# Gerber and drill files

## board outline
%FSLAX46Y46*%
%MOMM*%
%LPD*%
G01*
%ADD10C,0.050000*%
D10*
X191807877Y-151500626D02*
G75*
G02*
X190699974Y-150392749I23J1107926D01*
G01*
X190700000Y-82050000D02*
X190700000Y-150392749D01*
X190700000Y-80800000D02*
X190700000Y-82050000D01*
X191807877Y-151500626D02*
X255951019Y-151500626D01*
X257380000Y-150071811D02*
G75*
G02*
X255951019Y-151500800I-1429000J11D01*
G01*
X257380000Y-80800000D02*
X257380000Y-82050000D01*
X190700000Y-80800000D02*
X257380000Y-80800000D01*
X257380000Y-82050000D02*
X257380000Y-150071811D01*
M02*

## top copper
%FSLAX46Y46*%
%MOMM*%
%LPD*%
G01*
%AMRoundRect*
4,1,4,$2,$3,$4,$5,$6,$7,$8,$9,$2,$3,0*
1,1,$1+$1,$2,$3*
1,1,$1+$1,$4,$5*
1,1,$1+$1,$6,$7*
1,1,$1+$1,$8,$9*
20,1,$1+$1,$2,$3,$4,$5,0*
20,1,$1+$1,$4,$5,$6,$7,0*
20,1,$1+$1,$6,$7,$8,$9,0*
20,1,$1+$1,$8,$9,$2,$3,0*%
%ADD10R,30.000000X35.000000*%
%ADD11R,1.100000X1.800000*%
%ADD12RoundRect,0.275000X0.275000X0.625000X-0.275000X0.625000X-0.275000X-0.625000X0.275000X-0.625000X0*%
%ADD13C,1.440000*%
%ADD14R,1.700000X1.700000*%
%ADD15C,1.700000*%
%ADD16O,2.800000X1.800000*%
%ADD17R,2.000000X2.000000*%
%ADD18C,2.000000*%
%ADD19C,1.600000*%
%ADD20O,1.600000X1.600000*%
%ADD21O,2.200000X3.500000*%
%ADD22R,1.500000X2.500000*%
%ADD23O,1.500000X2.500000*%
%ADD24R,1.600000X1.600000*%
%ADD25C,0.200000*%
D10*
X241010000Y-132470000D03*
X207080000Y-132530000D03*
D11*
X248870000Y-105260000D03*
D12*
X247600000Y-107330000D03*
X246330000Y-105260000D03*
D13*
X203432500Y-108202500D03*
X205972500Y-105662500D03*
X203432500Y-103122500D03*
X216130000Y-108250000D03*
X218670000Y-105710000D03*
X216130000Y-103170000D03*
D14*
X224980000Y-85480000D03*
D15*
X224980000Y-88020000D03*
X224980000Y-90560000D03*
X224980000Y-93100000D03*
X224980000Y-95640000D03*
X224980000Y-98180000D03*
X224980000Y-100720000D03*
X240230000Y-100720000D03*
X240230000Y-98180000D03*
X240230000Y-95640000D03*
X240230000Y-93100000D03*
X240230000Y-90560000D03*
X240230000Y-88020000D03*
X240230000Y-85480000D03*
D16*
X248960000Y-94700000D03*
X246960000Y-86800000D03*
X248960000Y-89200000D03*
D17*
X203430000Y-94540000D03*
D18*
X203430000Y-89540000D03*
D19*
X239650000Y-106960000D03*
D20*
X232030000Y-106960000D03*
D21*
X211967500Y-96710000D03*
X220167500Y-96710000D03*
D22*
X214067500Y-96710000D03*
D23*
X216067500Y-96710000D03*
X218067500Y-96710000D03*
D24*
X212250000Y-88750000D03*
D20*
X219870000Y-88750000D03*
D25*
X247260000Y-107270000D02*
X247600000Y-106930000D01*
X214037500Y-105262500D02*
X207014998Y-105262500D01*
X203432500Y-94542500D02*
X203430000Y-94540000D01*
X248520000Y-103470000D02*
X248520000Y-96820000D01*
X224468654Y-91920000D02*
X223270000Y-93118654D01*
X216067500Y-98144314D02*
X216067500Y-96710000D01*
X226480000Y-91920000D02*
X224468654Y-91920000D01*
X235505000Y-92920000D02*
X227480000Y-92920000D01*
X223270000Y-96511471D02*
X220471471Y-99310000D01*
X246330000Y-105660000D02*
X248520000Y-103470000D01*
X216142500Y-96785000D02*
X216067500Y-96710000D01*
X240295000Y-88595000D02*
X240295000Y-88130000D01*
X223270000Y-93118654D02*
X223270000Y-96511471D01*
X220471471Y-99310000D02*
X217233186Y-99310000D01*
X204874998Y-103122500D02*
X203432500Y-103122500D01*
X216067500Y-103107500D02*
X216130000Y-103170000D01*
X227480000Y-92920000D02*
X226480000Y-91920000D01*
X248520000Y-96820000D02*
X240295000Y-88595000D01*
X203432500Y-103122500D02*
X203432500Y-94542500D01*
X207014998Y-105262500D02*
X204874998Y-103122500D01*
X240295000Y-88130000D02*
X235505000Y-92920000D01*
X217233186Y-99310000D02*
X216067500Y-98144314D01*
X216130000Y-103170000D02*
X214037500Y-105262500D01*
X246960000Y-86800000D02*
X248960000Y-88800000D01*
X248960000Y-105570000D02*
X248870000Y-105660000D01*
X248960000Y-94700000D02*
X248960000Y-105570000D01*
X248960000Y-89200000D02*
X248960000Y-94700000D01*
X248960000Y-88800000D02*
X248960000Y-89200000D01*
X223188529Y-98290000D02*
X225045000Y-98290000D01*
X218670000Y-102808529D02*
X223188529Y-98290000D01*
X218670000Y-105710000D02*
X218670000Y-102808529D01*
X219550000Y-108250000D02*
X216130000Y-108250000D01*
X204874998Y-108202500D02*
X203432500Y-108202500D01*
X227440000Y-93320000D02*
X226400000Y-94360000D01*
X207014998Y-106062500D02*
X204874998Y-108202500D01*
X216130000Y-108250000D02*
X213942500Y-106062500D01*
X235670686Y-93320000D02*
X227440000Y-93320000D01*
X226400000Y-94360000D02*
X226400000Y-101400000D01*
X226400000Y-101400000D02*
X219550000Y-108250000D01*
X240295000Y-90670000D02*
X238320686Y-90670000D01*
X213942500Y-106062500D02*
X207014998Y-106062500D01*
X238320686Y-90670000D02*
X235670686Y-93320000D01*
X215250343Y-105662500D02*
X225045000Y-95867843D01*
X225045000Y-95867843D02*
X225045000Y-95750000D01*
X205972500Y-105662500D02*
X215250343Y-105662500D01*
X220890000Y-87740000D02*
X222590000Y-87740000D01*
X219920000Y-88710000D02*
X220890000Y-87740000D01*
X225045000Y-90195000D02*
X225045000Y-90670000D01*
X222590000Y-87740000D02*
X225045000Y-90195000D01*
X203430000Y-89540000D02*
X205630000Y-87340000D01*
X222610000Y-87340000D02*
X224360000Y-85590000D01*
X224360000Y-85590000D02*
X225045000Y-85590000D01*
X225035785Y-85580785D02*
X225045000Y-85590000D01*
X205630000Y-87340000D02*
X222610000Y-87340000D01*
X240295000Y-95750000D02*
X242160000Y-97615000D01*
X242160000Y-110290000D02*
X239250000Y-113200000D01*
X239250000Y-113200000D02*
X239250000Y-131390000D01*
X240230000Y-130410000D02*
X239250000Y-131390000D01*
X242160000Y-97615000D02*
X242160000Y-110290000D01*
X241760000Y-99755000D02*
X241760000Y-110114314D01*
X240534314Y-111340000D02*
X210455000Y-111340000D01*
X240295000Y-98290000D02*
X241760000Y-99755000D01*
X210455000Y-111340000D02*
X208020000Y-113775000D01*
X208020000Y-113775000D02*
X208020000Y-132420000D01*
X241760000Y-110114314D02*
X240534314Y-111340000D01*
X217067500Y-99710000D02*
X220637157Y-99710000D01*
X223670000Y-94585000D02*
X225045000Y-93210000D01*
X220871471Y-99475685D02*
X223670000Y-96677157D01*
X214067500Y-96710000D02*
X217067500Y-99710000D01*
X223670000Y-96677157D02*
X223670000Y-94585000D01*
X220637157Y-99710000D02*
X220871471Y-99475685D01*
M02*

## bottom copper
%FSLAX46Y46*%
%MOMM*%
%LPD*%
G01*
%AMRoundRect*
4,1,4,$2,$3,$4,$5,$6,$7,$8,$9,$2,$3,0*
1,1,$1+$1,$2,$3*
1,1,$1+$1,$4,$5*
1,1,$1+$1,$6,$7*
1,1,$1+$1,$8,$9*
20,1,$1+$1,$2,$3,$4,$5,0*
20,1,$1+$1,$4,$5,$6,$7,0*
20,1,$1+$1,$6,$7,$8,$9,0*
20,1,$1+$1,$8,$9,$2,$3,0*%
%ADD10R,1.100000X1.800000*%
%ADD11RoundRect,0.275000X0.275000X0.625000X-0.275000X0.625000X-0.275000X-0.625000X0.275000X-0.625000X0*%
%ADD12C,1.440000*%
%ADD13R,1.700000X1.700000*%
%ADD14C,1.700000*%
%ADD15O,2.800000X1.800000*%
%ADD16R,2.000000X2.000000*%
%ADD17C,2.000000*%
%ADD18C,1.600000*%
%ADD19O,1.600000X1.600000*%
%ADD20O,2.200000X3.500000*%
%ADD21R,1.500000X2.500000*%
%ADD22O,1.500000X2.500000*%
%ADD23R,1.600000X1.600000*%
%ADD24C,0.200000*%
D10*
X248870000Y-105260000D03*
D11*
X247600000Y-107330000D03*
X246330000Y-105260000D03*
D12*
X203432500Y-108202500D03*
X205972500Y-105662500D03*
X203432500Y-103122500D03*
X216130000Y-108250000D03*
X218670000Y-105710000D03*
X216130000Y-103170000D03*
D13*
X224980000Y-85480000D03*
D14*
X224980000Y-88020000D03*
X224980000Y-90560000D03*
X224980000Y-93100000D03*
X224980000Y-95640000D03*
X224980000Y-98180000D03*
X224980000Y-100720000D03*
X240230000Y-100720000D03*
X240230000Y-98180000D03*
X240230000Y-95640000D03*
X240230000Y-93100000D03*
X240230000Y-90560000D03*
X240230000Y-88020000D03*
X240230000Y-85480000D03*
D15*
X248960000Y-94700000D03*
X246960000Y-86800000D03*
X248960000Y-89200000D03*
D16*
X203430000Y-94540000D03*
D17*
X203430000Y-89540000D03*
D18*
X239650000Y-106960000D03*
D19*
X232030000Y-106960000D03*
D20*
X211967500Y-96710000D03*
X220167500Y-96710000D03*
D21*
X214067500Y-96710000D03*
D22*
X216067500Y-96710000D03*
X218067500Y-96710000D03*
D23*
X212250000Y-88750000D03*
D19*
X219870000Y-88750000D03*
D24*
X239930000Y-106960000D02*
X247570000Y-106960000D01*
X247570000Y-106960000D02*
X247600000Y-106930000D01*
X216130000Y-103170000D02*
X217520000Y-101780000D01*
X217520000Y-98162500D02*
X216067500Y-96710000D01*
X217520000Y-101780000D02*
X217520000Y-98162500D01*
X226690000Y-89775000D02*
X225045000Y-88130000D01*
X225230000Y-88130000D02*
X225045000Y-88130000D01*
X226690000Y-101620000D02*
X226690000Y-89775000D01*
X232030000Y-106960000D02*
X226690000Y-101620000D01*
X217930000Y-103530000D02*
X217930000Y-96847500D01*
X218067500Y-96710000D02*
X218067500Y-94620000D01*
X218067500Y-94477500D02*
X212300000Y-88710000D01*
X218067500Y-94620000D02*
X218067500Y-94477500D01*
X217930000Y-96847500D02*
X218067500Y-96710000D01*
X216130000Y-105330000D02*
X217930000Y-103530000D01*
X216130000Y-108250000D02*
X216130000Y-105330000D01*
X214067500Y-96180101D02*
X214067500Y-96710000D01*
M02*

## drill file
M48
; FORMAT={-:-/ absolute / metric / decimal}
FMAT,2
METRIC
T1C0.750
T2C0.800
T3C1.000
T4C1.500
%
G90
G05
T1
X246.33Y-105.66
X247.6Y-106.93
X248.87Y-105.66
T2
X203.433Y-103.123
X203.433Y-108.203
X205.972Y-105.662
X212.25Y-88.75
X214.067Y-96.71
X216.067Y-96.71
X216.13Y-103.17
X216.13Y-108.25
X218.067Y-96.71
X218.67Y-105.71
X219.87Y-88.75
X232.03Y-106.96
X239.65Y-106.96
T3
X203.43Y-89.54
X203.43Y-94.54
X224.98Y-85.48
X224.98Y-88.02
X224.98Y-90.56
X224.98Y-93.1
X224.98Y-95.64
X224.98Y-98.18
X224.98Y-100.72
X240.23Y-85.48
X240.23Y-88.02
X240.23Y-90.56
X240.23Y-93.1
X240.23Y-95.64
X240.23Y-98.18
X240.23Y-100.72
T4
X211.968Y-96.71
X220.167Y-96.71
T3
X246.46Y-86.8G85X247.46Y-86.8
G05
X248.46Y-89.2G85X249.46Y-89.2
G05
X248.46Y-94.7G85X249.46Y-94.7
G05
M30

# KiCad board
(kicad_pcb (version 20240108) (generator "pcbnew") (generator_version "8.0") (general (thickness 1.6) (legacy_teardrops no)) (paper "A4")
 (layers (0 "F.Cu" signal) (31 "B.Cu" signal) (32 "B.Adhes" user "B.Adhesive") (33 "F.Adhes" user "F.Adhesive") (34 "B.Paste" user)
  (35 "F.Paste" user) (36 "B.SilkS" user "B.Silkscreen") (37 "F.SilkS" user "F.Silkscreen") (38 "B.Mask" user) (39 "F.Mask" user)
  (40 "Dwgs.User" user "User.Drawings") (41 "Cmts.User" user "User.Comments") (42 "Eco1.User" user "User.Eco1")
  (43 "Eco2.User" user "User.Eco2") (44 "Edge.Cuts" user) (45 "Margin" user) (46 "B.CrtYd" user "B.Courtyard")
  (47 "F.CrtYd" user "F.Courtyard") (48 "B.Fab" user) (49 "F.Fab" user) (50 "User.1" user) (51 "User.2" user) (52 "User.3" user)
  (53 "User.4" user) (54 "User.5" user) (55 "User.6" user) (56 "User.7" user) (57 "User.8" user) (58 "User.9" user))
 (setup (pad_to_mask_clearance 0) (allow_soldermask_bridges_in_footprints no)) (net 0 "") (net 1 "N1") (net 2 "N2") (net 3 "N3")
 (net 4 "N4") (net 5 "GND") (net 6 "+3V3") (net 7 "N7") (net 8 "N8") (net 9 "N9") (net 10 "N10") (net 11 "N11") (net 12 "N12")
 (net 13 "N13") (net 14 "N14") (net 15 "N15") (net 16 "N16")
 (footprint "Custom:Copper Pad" (layer "F.Cu") (at 249.51 111.47)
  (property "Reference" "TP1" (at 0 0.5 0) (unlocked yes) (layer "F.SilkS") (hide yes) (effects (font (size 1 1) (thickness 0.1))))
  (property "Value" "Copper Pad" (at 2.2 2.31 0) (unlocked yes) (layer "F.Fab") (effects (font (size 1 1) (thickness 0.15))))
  (pad "1" smd rect (at -8.5 21) (size 30 35) (layers "F.Cu") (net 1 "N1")))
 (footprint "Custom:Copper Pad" (layer "F.Cu") (at 212.58 112.03)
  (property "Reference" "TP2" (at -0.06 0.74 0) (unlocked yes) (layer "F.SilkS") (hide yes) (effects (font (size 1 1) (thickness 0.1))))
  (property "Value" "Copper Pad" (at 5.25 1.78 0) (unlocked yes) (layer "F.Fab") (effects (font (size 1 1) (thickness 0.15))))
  (pad "1" smd rect (at -5.5 20.5) (size 30 35) (layers "F.Cu") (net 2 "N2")))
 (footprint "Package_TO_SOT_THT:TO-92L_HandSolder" (layer "F.Cu") (at 248.87 105.66 180)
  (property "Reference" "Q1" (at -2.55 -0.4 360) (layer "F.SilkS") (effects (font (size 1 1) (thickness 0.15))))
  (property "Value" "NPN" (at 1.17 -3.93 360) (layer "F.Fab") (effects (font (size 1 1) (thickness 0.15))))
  (pad "1" thru_hole rect (at 0 0 180) (size 1.1 1.8) (drill 0.75 (offset 0 0.4)) (layers "*.Cu" "*.Mask") (remove_unused_layers no)
   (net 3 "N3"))
  (pad "2" thru_hole roundrect (at 1.27 -1.27 180) (size 1.1 1.8) (drill 0.75 (offset 0 -0.4)) (layers "*.Cu" "*.Mask")
   (remove_unused_layers no) (roundrect_rratio 0.25) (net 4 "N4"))
  (pad "3" thru_hole roundrect (at 2.54 0 180) (size 1.1 1.8) (drill 0.75 (offset 0 0.4)) (layers "*.Cu" "*.Mask") (remove_unused_layers no)
   (roundrect_rratio 0.25) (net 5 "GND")))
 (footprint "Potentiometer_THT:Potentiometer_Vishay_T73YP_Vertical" (layer "F.Cu") (at 203.4325 108.2025)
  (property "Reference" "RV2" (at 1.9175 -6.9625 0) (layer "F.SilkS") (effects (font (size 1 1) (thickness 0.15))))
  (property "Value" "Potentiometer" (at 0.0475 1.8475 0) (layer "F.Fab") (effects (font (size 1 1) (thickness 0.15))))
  (pad "1" thru_hole circle (at 0 0) (size 1.44 1.44) (drill 0.8) (layers "*.Cu" "*.Mask") (remove_unused_layers no) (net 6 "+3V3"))
  (pad "2" thru_hole circle (at 2.54 -2.54) (size 1.44 1.44) (drill 0.8) (layers "*.Cu" "*.Mask") (remove_unused_layers no) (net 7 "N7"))
  (pad "3" thru_hole circle (at 0 -5.08) (size 1.44 1.44) (drill 0.8) (layers "*.Cu" "*.Mask") (remove_unused_layers no) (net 5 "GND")))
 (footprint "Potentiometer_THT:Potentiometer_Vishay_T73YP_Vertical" (layer "F.Cu") (at 216.13 108.25)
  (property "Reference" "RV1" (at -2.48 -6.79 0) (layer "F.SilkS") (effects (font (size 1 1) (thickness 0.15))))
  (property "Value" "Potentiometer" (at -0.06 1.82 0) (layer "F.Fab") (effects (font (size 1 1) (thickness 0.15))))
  (pad "1" thru_hole circle (at 0 0) (size 1.44 1.44) (drill 0.8) (layers "*.Cu" "*.Mask") (remove_unused_layers no) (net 6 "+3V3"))
  (pad "2" thru_hole circle (at 2.54 -2.54) (size 1.44 1.44) (drill 0.8) (layers "*.Cu" "*.Mask") (remove_unused_layers no) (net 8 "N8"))
  (pad "3" thru_hole circle (at 0 -5.08) (size 1.44 1.44) (drill 0.8) (layers "*.Cu" "*.Mask") (remove_unused_layers no) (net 5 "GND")))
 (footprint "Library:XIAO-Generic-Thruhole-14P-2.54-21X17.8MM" (layer "F.Cu") (at 232.605 93.1)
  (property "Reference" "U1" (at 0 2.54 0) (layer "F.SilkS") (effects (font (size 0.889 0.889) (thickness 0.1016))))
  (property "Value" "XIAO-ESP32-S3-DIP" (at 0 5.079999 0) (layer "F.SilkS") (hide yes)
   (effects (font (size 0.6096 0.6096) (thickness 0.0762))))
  (pad "1" thru_hole rect (at -7.625 -7.62 180) (size 1.7 1.7) (drill 1) (layers "*.Cu" "*.Mask") (remove_unused_layers no) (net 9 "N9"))
  (pad "2" thru_hole circle (at -7.625 -5.08 180) (size 1.7 1.7) (drill 1) (layers "*.Cu" "*.Mask") (remove_unused_layers no) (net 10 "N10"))
  (pad "3" thru_hole circle (at -7.625 -2.54 180) (size 1.7 1.7) (drill 1) (layers "*.Cu" "*.Mask") (remove_unused_layers no) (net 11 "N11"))
  (pad "4" thru_hole circle (at -7.625 0 180) (size 1.7 1.7) (drill 1) (layers "*.Cu" "*.Mask") (remove_unused_layers no) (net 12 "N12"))
  (pad "5" thru_hole circle (at -7.625 2.54 180) (size 1.7 1.7) (drill 1) (layers "*.Cu" "*.Mask") (remove_unused_layers no) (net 7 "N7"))
  (pad "6" thru_hole circle (at -7.625 5.08) (size 1.7 1.7) (drill 1) (layers "*.Cu" "*.Mask") (remove_unused_layers no) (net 8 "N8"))
  (pad "7" thru_hole circle (at -7.625 7.62 180) (size 1.7 1.7) (drill 1) (layers "*.Cu" "*.Mask") (remove_unused_layers no) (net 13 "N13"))
  (pad "8" thru_hole circle (at 7.625 7.62 180) (size 1.7 1.7) (drill 1) (layers "*.Cu" "*.Mask") (remove_unused_layers no) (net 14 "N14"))
  (pad "9" thru_hole circle (at 7.625 5.08 180) (size 1.7 1.7) (drill 1) (layers "*.Cu" "*.Mask") (remove_unused_layers no) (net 2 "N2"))
  (pad "10" thru_hole circle (at 7.625 2.54 180) (size 1.7 1.7) (drill 1) (layers "*.Cu" "*.Mask") (remove_unused_layers no) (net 1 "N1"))
  (pad "11" thru_hole circle (at 7.625 0 180) (size 1.7 1.7) (drill 1) (layers "*.Cu" "*.Mask") (remove_unused_layers no) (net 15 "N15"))
  (pad "12" thru_hole circle (at 7.625 -2.54 180) (size 1.7 1.7) (drill 1) (layers "*.Cu" "*.Mask") (remove_unused_layers no) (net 6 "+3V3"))
  (pad "13" thru_hole circle (at 7.625 -5.08 180) (size 1.7 1.7) (drill 1) (layers "*.Cu" "*.Mask") (remove_unused_layers no) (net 5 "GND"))
  (pad "14" thru_hole circle (at 7.625 -7.62 180) (size 1.7 1.7) (drill 1) (layers "*.Cu" "*.Mask") (remove_unused_layers no) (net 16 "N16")))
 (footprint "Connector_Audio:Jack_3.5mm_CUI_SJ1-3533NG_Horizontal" (layer "F.Cu") (at 246.96 86.8)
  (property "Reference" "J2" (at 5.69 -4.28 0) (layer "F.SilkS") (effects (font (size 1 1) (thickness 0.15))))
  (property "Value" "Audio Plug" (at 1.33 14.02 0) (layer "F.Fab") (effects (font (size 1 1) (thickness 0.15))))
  (pad "R" thru_hole oval (at 2 7.9) (size 2.8 1.8) (drill oval 2 1) (layers "*.Cu" "*.Mask") (remove_unused_layers no) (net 3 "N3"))
  (pad "S" thru_hole oval (at 0 0) (size 2.8 1.8) (drill oval 2 1) (layers "*.Cu" "*.Mask") (remove_unused_layers no) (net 3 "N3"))
  (pad "T" thru_hole oval (at 2 2.4) (size 2.8 1.8) (drill oval 2 1) (layers "*.Cu" "*.Mask") (remove_unused_layers no) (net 3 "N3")))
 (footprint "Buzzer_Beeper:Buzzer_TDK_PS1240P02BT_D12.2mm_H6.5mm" (layer "F.Cu") (at 203.43 94.54 90)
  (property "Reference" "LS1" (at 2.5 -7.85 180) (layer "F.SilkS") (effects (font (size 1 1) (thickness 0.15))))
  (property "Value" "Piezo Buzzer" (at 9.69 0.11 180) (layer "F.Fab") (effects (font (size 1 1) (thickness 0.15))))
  (pad "1" thru_hole rect (at 0 0 90) (size 2 2) (drill 1) (layers "*.Cu" "*.Mask") (remove_unused_layers no) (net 5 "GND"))
  (pad "2" thru_hole circle (at 5 0 90) (size 2 2) (drill 1) (layers "*.Cu" "*.Mask") (remove_unused_layers no) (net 9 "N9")))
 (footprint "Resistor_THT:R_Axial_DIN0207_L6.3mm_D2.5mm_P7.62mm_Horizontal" (layer "F.Cu") (at 239.65 106.96 180)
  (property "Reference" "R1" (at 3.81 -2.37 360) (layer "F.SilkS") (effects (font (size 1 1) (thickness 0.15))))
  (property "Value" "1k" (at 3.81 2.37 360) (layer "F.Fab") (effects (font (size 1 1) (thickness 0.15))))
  (pad "1" thru_hole circle (at 0 0 180) (size 1.6 1.6) (drill 0.8) (layers "*.Cu" "*.Mask") (remove_unused_layers no) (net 4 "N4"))
  (pad "2" thru_hole oval (at 7.62 0 180) (size 1.6 1.6) (drill 0.8) (layers "*.Cu" "*.Mask") (remove_unused_layers no) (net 10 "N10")))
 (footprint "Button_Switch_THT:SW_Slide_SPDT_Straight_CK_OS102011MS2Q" (layer "F.Cu") (at 214.0675 96.71)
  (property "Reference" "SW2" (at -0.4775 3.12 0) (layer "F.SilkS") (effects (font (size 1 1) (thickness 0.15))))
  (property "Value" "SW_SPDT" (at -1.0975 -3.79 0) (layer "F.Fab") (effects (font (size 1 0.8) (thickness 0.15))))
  (pad "" thru_hole oval (at -2.1 0) (size 2.2 3.5) (drill 1.5) (layers "*.Cu" "*.Mask") (remove_unused_layers no))
  (pad "" thru_hole oval (at 6.1 0) (size 2.2 3.5) (drill 1.5) (layers "*.Cu" "*.Mask") (remove_unused_layers no))
  (pad "1" thru_hole rect (at 0 0) (size 1.5 2.5) (drill 0.8) (layers "*.Cu" "*.Mask") (remove_unused_layers no) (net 12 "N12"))
  (pad "2" thru_hole oval (at 2 0) (size 1.5 2.5) (drill 0.8) (layers "*.Cu" "*.Mask") (remove_unused_layers no) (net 5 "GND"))
  (pad "3" thru_hole oval (at 4 0) (size 1.5 2.5) (drill 0.8) (layers "*.Cu" "*.Mask") (remove_unused_layers no) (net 6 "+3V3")))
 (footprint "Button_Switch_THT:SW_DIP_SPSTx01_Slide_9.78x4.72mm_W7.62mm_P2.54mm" (layer "F.Cu") (at 212.25 88.75)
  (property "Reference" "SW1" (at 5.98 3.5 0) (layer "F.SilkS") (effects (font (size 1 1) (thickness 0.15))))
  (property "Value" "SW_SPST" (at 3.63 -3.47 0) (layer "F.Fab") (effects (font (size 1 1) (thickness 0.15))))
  (pad "1" thru_hole rect (at 0 0) (size 1.6 1.6) (drill 0.8) (layers "*.Cu" "*.Mask") (remove_unused_layers no) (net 6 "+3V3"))
  (pad "2" thru_hole oval (at 7.62 0) (size 1.6 1.6) (drill 0.8) (layers "*.Cu" "*.Mask") (remove_unused_layers no) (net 11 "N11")))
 (gr_arc (start 191.807877 151.500626) (mid 191.02449 151.176136) (end 190.7 150.392749) (stroke (width 0.05) (type default))
  (layer "Edge.Cuts"))
 (gr_line (start 190.7 82.05) (end 190.7 150.392749) (stroke (width 0.05) (type default)) (layer "Edge.Cuts"))
 (gr_line (start 190.7 80.8) (end 190.7 82.05) (stroke (width 0.05) (type default)) (layer "Edge.Cuts"))
 (gr_line (start 191.807877 151.500626) (end 255.951019 151.500626) (stroke (width 0.05) (type default)) (layer "Edge.Cuts"))
 (gr_arc (start 257.38 150.071811) (mid 256.961461 151.082253) (end 255.951019 151.500792) (stroke (width 0.05) (type default))
  (layer "Edge.Cuts"))
 (gr_line (start 257.38 80.8) (end 257.38 82.05) (stroke (width 0.05) (type default)) (layer "Edge.Cuts"))
 (gr_line (start 190.7 80.8) (end 257.38 80.8) (stroke (width 0.05) (type default)) (layer "Edge.Cuts"))
 (gr_line (start 257.38 82.05) (end 257.38 150.071811) (stroke (width 0.05) (type default)) (layer "Edge.Cuts"))
 (segment (start 247.26 107.27) (end 247.6 106.93) (width 0.2) (layer "F.Cu") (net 4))
 (segment (start 239.93 106.96) (end 247.57 106.96) (width 0.2) (layer "B.Cu") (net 4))
 (segment (start 247.57 106.96) (end 247.6 106.93) (width 0.2) (layer "B.Cu") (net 4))
 (segment (start 214.0375 105.2625) (end 207.014998 105.2625) (width 0.2) (layer "F.Cu") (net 5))
 (segment (start 203.4325 94.5425) (end 203.43 94.54) (width 0.2) (layer "F.Cu") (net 5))
 (segment (start 248.52 103.47) (end 248.52 96.82) (width 0.2) (layer "F.Cu") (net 5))
 (segment (start 224.468654 91.92) (end 223.27 93.118654) (width 0.2) (layer "F.Cu") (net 5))
 (segment (start 216.0675 98.144314) (end 216.0675 96.71) (width 0.2) (layer "F.Cu") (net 5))
 (segment (start 226.48 91.92) (end 224.468654 91.92) (width 0.2) (layer "F.Cu") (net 5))
 (segment (start 235.505 92.92) (end 227.48 92.92) (width 0.2) (layer "F.Cu") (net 5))
 (segment (start 223.27 96.511471) (end 220.471471 99.31) (width 0.2) (layer "F.Cu") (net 5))
 (segment (start 246.33 105.66) (end 248.52 103.47) (width 0.2) (layer "F.Cu") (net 5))
 (segment (start 216.1425 96.785) (end 216.0675 96.71) (width 0.2) (layer "F.Cu") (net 5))
 (segment (start 240.295 88.595) (end 240.295 88.13) (width 0.2) (layer "F.Cu") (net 5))
 (segment (start 223.27 93.118654) (end 223.27 96.511471) (width 0.2) (layer "F.Cu") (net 5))
 (segment (start 220.471471 99.31) (end 217.233186 99.31) (width 0.2) (layer "F.Cu") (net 5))
 (segment (start 204.874998 103.1225) (end 203.4325 103.1225) (width 0.2) (layer "F.Cu") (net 5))
 (segment (start 216.0675 103.1075) (end 216.13 103.17) (width 0.2) (layer "F.Cu") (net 5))
 (segment (start 227.48 92.92) (end 226.48 91.92) (width 0.2) (layer "F.Cu") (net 5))
 (segment (start 248.52 96.82) (end 240.295 88.595) (width 0.2) (layer "F.Cu") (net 5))
 (segment (start 203.4325 103.1225) (end 203.4325 94.5425) (width 0.2) (layer "F.Cu") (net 5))
 (segment (start 207.014998 105.2625) (end 204.874998 103.1225) (width 0.2) (layer "F.Cu") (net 5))
 (segment (start 240.295 88.13) (end 235.505 92.92) (width 0.2) (layer "F.Cu") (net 5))
 (segment (start 217.233186 99.31) (end 216.0675 98.144314) (width 0.2) (layer "F.Cu") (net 5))
 (segment (start 216.13 103.17) (end 214.0375 105.2625) (width 0.2) (layer "F.Cu") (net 5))
 (segment (start 216.13 103.17) (end 217.52 101.78) (width 0.2) (layer "B.Cu") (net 5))
 (segment (start 217.52 98.1625) (end 216.0675 96.71) (width 0.2) (layer "B.Cu") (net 5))
 (segment (start 217.52 101.78) (end 217.52 98.1625) (width 0.2) (layer "B.Cu") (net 5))
 (segment (start 246.96 86.8) (end 248.96 88.8) (width 0.2) (layer "F.Cu") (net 3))
 (segment (start 248.96 105.57) (end 248.87 105.66) (width 0.2) (layer "F.Cu") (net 3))
 (segment (start 248.96 94.7) (end 248.96 105.57) (width 0.2) (layer "F.Cu") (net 3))
 (segment (start 248.96 89.2) (end 248.96 94.7) (width 0.2) (layer "F.Cu") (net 3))
 (segment (start 248.96 88.8) (end 248.96 89.2) (width 0.2) (layer "F.Cu") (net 3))
 (segment (start 226.69 89.775) (end 225.045 88.13) (width 0.2) (layer "B.Cu") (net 10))
 (segment (start 225.23 88.13) (end 225.045 88.13) (width 0.2) (layer "B.Cu") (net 10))
 (segment (start 226.69 101.62) (end 226.69 89.775) (width 0.2) (layer "B.Cu") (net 10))
 (segment (start 232.03 106.96) (end 226.69 101.62) (width 0.2) (layer "B.Cu") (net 10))
 (segment (start 223.188529 98.29) (end 225.045 98.29) (width 0.2) (layer "F.Cu") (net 8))
 (segment (start 218.67 102.808529) (end 223.188529 98.29) (width 0.2) (layer "F.Cu") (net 8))
 (segment (start 218.67 105.71) (end 218.67 102.808529) (width 0.2) (layer "F.Cu") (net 8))
 (segment (start 219.55 108.25) (end 216.13 108.25) (width 0.2) (layer "F.Cu") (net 6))
 (segment (start 204.874998 108.2025) (end 203.4325 108.2025) (width 0.2) (layer "F.Cu") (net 6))
 (segment (start 227.44 93.32) (end 226.4 94.36) (width 0.2) (layer "F.Cu") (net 6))
 (segment (start 207.014998 106.0625) (end 204.874998 108.2025) (width 0.2) (layer "F.Cu") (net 6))
 (segment (start 216.13 108.25) (end 213.9425 106.0625) (width 0.2) (layer "F.Cu") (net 6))
 (segment (start 235.670686 93.32) (end 227.44 93.32) (width 0.2) (layer "F.Cu") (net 6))
 (segment (start 226.4 94.36) (end 226.4 101.4) (width 0.2) (layer "F.Cu") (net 6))
 (segment (start 226.4 101.4) (end 219.55 108.25) (width 0.2) (layer "F.Cu") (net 6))
 (segment (start 240.295 90.67) (end 238.320686 90.67) (width 0.2) (layer "F.Cu") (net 6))
 (segment (start 213.9425 106.0625) (end 207.014998 106.0625) (width 0.2) (layer "F.Cu") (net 6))
 (segment (start 238.320686 90.67) (end 235.670686 93.32) (width 0.2) (layer "F.Cu") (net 6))
 (segment (start 217.93 103.53) (end 217.93 96.8475) (width 0.2) (layer "B.Cu") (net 6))
 (segment (start 218.0675 96.71) (end 218.0675 94.62) (width 0.2) (layer "B.Cu") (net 6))
 (segment (start 218.0675 94.4775) (end 212.3 88.71) (width 0.2) (layer "B.Cu") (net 6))
 (segment (start 218.0675 94.62) (end 218.0675 94.4775) (width 0.2) (layer "B.Cu") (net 6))
 (segment (start 217.93 96.8475) (end 218.0675 96.71) (width 0.2) (layer "B.Cu") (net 6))
 (segment (start 216.13 105.33) (end 217.93 103.53) (width 0.2) (layer "B.Cu") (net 6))
 (segment (start 216.13 108.25) (end 216.13 105.33) (width 0.2) (layer "B.Cu") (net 6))
 (segment (start 215.250343 105.6625) (end 225.045 95.867843) (width 0.2) (layer "F.Cu") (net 7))
 (segment (start 225.045 95.867843) (end 225.045 95.75) (width 0.2) (layer "F.Cu") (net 7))
 (segment (start 205.9725 105.6625) (end 215.250343 105.6625) (width 0.2) (layer "F.Cu") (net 7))
 (segment (start 220.89 87.74) (end 222.59 87.74) (width 0.2) (layer "F.Cu") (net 11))
 (segment (start 219.92 88.71) (end 220.89 87.74) (width 0.2) (layer "F.Cu") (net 11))
 (segment (start 225.045 90.195) (end 225.045 90.67) (width 0.2) (layer "F.Cu") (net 11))
 (segment (start 222.59 87.74) (end 225.045 90.195) (width 0.2) (layer "F.Cu") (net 11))
 (segment (start 203.43 89.54) (end 205.63 87.34) (width 0.2) (layer "F.Cu") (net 9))
 (segment (start 222.61 87.34) (end 224.36 85.59) (width 0.2) (layer "F.Cu") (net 9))
 (segment (start 224.36 85.59) (end 225.045 85.59) (width 0.2) (layer "F.Cu") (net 9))
 (segment (start 225.035785 85.580785) (end 225.045 85.59) (width 0.2) (layer "F.Cu") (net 9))
 (segment (start 205.63 87.34) (end 222.61 87.34) (width 0.2) (layer "F.Cu") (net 9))
 (segment (start 240.295 95.75) (end 242.16 97.615) (width 0.2) (layer "F.Cu") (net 1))
 (segment (start 242.16 110.29) (end 239.25 113.2) (width 0.2) (layer "F.Cu") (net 1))
 (segment (start 239.25 113.2) (end 239.25 131.39) (width 0.2) (layer "F.Cu") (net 1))
 (segment (start 240.23 130.41) (end 239.25 131.39) (width 0.2) (layer "F.Cu") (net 1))
 (segment (start 242.16 97.615) (end 242.16 110.29) (width 0.2) (layer "F.Cu") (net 1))
 (segment (start 241.76 99.755) (end 241.76 110.114314) (width 0.2) (layer "F.Cu") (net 2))
 (segment (start 240.534314 111.34) (end 210.455 111.34) (width 0.2) (layer "F.Cu") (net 2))
 (segment (start 240.295 98.29) (end 241.76 99.755) (width 0.2) (layer "F.Cu") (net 2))
 (segment (start 210.455 111.34) (end 208.02 113.775) (width 0.2) (layer "F.Cu") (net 2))
 (segment (start 208.02 113.775) (end 208.02 132.42) (width 0.2) (layer "F.Cu") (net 2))
 (segment (start 241.76 110.114314) (end 240.534314 111.34) (width 0.2) (layer "F.Cu") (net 2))
 (segment (start 217.0675 99.71) (end 220.637157 99.71) (width 0.2) (layer "F.Cu") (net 12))
 (segment (start 223.67 94.585) (end 225.045 93.21) (width 0.2) (layer "F.Cu") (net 12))
 (segment (start 220.871471 99.475685) (end 223.67 96.677157) (width 0.2) (layer "F.Cu") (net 12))
 (segment (start 214.0675 96.71) (end 217.0675 99.71) (width 0.2) (layer "F.Cu") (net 12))
 (segment (start 223.67 96.677157) (end 223.67 94.585) (width 0.2) (layer "F.Cu") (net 12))
 (segment (start 220.637157 99.71) (end 220.871471 99.475685) (width 0.2) (layer "F.Cu") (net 12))
 (segment (start 214.0675 96.180101) (end 214.0675 96.71) (width 0.2) (layer "B.Cu") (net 12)))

